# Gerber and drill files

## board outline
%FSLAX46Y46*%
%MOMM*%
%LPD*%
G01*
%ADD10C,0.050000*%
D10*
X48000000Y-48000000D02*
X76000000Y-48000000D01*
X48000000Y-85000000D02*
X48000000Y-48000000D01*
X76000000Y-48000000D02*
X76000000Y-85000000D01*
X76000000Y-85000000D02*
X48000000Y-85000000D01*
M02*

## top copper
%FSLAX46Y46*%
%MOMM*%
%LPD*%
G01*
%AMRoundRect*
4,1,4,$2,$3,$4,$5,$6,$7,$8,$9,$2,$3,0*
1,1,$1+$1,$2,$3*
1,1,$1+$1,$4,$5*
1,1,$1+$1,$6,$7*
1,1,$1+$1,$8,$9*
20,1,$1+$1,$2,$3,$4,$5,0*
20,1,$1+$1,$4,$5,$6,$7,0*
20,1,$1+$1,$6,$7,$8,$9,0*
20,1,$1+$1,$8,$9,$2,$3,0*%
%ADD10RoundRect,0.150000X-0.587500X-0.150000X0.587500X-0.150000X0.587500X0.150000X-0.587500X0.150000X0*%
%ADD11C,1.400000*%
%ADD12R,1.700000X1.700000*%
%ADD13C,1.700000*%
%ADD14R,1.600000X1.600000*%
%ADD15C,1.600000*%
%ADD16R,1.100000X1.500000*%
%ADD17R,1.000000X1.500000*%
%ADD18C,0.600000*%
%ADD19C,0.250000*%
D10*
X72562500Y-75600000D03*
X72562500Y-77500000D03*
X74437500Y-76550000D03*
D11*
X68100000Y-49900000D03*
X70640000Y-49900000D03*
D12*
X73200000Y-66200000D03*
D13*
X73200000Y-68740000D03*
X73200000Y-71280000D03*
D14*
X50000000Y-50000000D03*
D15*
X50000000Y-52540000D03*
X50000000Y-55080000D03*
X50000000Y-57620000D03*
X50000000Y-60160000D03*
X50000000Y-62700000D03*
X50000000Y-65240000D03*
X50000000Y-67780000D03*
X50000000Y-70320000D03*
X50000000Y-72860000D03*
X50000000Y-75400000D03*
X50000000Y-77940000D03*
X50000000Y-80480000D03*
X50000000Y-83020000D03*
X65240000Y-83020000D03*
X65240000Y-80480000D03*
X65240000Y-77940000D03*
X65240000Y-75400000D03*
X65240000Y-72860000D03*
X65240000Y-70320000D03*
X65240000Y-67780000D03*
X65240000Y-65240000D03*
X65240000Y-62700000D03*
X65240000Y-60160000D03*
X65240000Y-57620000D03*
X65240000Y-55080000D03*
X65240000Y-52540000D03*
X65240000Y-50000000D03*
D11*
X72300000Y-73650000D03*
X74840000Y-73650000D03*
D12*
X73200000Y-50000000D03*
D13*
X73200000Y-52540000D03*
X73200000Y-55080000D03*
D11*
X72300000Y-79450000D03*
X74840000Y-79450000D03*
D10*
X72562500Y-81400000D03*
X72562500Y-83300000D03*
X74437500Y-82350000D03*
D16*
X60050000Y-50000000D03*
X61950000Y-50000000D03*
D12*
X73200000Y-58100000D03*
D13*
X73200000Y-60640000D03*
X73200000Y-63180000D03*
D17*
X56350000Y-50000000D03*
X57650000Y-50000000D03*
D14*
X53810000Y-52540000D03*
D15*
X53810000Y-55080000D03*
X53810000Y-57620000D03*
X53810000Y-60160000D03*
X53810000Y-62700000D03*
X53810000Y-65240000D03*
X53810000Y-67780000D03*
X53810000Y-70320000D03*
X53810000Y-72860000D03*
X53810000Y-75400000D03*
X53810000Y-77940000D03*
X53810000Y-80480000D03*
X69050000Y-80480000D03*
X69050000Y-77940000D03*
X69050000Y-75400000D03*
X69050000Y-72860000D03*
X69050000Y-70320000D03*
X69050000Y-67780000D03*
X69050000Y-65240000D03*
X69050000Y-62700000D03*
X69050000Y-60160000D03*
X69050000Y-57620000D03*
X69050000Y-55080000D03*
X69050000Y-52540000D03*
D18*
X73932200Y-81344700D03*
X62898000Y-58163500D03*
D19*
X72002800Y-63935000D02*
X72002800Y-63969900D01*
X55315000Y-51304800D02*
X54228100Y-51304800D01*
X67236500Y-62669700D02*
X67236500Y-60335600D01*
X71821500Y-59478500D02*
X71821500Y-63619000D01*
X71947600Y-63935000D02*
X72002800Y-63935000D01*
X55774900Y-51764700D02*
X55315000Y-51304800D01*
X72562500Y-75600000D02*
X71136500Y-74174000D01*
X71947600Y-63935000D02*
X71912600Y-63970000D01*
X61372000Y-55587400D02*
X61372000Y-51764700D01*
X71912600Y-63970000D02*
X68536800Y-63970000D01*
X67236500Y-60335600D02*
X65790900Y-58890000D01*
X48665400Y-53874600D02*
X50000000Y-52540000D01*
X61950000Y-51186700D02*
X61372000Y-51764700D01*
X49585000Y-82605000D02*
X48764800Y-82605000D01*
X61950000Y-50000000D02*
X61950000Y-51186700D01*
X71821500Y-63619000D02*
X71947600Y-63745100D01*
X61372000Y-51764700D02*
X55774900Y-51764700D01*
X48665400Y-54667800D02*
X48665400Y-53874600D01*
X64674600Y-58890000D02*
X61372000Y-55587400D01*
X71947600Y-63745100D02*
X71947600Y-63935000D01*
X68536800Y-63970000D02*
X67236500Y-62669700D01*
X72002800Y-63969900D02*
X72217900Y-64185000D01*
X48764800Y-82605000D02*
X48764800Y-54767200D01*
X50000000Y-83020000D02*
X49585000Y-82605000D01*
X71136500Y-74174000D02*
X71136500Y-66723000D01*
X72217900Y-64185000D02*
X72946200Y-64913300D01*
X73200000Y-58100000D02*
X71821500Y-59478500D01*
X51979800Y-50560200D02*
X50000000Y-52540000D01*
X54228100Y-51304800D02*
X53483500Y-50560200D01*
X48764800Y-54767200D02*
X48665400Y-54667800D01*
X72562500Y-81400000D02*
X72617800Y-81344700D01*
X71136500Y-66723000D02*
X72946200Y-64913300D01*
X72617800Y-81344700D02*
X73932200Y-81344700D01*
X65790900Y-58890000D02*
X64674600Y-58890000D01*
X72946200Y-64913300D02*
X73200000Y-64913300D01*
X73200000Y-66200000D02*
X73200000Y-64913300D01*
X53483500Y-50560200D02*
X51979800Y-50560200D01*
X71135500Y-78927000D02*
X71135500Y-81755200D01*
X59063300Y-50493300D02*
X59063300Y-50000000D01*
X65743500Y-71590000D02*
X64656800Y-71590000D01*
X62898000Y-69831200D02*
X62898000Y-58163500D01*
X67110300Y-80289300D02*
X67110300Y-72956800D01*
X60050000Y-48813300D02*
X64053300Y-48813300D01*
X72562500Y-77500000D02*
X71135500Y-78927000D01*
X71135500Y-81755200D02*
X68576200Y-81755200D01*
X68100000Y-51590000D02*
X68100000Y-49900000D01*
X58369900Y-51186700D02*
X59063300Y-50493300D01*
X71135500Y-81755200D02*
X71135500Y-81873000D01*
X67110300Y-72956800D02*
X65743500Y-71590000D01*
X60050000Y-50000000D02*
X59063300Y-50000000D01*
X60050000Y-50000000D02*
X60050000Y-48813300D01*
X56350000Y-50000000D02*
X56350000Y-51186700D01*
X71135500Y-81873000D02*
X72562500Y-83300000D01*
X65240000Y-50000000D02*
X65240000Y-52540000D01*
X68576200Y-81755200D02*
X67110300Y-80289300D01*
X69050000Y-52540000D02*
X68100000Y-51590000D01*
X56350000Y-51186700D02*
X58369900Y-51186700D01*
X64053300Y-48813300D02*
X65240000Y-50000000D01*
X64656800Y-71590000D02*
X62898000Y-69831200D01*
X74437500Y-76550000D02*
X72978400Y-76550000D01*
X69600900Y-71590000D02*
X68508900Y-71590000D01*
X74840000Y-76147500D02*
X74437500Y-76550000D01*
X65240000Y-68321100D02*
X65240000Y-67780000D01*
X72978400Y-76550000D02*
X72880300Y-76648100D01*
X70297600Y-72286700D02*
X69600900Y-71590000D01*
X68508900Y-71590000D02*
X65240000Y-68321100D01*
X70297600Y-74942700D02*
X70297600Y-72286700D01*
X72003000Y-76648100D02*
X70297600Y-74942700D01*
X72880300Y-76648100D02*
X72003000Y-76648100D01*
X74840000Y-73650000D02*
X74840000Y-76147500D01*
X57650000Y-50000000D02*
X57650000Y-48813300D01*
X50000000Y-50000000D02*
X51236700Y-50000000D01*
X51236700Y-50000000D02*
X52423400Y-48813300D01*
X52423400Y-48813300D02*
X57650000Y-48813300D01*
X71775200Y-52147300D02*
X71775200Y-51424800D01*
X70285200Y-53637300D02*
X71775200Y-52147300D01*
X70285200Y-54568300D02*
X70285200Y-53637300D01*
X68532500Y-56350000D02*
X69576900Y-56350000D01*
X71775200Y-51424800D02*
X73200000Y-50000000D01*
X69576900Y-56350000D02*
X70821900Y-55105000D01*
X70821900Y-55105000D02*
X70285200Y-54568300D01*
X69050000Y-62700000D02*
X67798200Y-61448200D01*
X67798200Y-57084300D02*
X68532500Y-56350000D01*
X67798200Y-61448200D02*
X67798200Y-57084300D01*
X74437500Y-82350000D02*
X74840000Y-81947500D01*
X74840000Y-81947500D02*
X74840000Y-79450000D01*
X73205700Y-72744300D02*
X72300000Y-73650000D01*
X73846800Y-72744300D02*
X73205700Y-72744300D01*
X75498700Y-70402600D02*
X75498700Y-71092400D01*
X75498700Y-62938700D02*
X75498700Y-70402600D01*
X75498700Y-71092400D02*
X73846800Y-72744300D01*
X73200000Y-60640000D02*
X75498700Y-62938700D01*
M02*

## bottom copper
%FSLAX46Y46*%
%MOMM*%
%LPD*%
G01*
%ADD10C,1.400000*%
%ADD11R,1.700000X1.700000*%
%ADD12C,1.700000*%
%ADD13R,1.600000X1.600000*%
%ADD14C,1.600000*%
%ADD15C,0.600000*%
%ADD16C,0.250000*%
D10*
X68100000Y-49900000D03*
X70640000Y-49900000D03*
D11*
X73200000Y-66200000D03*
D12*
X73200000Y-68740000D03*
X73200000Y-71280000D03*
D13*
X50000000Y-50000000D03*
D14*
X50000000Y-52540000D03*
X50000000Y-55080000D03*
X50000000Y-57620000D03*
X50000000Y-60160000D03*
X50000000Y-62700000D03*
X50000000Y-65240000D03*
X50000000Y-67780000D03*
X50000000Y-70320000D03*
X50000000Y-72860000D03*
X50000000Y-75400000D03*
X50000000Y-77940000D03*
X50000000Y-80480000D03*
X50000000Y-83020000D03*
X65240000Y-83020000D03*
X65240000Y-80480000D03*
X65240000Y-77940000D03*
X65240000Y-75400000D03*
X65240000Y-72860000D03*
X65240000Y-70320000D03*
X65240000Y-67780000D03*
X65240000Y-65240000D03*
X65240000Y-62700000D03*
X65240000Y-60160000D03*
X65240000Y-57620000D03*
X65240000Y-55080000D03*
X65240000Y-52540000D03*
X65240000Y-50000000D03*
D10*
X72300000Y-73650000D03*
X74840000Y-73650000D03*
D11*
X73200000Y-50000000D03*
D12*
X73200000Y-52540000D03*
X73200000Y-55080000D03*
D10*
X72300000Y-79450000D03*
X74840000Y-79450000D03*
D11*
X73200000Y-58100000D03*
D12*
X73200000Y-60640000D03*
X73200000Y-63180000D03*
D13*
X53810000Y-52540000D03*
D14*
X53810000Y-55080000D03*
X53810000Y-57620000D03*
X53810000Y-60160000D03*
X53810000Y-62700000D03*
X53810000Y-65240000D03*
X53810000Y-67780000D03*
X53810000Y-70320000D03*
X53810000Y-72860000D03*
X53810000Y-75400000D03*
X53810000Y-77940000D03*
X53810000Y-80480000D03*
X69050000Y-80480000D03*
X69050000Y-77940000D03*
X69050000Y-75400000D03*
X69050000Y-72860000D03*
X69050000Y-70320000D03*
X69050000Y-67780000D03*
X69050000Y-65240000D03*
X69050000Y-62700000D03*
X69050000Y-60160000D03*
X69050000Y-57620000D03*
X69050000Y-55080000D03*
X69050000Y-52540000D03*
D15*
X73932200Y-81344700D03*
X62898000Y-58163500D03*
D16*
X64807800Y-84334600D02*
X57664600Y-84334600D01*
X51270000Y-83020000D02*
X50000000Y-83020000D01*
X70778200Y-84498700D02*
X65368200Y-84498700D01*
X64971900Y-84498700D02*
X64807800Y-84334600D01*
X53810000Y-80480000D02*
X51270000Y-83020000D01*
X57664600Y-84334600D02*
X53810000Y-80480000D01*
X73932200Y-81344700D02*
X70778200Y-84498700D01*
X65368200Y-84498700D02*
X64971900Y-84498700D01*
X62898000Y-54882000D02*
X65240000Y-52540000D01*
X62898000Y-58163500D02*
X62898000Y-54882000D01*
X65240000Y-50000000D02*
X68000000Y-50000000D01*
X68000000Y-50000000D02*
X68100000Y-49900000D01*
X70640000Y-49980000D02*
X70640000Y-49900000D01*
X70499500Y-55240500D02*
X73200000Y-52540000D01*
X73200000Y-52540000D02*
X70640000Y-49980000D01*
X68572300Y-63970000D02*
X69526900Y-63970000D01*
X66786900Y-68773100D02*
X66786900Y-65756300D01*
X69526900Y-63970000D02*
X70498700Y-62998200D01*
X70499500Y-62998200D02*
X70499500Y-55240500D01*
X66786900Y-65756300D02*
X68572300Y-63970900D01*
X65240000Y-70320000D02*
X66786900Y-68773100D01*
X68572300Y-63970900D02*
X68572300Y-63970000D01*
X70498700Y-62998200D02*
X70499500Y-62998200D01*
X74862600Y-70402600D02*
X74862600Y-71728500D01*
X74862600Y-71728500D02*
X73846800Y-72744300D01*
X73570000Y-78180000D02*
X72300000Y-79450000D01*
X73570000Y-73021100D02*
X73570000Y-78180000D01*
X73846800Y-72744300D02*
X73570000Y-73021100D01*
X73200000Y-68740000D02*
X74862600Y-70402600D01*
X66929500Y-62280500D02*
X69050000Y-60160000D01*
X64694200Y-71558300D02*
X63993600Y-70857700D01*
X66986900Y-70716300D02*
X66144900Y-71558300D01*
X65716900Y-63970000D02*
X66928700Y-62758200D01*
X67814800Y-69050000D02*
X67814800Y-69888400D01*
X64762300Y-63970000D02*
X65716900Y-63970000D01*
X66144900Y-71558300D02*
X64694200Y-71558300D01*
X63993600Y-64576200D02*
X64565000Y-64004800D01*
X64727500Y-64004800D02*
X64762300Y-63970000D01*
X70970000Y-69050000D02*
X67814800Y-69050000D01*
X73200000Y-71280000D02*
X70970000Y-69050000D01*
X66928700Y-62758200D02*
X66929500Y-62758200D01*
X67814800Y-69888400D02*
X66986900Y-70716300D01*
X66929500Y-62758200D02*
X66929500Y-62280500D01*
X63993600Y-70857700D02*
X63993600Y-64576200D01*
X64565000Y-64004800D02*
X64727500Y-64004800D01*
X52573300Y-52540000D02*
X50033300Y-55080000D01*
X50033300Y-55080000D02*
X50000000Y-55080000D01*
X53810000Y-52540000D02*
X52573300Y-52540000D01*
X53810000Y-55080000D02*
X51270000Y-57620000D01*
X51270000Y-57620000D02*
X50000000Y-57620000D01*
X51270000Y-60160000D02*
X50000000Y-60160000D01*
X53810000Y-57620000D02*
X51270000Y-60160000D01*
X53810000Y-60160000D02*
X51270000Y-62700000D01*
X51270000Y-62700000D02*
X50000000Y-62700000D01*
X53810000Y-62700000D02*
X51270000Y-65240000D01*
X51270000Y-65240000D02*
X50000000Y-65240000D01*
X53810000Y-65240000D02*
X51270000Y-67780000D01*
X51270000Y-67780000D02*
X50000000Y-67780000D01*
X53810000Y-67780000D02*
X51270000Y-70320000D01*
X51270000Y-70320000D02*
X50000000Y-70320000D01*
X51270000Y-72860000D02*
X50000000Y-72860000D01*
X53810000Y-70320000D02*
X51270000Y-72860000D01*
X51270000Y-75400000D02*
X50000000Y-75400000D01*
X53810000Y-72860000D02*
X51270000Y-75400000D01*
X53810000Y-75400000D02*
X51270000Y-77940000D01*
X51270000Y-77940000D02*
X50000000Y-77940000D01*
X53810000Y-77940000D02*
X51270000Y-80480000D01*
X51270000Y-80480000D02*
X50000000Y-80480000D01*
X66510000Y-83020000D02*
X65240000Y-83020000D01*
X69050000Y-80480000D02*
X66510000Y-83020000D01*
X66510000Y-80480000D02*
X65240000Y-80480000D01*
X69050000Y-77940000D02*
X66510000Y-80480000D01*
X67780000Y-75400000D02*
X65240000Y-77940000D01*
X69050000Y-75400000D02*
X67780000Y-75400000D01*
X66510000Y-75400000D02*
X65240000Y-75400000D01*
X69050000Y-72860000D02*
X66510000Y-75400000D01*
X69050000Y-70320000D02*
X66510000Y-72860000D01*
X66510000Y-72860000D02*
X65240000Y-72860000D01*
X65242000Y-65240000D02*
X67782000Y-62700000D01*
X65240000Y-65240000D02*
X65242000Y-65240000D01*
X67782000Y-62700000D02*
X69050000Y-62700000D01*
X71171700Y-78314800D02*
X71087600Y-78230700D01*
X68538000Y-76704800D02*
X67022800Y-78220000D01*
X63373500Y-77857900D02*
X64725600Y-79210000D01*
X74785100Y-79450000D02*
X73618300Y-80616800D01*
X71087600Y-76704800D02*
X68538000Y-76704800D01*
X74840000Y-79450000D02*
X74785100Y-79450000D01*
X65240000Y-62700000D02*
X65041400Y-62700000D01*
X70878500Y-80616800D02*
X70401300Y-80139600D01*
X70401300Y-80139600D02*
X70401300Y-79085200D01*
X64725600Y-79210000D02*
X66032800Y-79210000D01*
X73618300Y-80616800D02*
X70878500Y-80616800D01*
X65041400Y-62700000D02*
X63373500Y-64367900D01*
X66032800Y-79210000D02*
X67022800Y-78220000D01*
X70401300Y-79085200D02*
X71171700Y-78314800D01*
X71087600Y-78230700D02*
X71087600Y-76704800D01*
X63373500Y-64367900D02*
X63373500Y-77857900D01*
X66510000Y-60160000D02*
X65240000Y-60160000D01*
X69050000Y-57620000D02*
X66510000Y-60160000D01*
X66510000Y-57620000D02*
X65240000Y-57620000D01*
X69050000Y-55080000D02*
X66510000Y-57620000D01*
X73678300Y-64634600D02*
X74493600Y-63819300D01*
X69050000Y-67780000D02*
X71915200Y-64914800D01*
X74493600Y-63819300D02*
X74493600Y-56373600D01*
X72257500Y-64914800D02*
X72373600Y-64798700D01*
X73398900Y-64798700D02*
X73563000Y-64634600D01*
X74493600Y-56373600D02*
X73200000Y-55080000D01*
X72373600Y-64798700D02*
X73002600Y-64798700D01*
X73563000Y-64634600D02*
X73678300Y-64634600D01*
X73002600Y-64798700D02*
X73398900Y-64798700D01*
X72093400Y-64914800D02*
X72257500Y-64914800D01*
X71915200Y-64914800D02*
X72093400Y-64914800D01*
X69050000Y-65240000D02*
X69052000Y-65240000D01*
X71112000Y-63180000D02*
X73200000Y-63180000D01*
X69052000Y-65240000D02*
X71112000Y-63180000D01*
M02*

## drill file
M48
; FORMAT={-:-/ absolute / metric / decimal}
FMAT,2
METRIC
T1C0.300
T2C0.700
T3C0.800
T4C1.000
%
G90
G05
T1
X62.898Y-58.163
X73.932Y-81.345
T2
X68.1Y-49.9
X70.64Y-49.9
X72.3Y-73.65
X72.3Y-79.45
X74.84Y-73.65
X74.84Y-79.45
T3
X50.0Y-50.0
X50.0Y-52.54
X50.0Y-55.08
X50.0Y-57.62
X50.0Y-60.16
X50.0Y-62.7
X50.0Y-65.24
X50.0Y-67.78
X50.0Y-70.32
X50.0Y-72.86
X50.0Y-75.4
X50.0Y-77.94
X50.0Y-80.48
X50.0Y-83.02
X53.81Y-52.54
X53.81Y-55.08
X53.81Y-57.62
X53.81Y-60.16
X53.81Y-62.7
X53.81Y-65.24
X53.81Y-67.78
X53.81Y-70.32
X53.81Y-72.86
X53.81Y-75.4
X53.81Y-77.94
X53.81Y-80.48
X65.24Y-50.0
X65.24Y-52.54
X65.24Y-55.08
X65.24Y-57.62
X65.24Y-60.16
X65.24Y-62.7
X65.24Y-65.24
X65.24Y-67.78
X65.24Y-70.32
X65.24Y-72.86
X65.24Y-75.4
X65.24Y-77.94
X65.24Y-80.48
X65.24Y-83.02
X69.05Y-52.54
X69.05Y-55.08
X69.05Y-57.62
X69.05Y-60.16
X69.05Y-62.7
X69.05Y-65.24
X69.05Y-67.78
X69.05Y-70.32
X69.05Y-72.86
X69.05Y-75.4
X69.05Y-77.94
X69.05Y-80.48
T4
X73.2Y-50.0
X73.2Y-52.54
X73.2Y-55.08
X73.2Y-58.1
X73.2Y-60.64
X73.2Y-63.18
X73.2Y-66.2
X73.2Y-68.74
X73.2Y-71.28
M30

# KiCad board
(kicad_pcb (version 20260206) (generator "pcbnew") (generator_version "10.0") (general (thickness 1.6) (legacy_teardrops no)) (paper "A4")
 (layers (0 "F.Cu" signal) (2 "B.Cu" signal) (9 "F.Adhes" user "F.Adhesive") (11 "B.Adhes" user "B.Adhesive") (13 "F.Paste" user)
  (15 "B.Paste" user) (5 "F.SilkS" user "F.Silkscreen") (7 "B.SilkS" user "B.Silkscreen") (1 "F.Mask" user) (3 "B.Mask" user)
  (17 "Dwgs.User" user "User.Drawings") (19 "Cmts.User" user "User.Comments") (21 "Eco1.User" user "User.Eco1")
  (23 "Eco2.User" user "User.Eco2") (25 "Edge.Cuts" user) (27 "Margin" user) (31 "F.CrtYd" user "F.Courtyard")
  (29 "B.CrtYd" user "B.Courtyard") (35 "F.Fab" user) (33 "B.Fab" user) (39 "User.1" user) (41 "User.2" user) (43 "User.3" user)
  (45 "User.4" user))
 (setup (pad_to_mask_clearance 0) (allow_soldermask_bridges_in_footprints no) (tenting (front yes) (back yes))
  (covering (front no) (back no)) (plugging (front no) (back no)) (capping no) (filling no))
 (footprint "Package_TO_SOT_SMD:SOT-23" (layer "F.Cu") (at 73.5 76.55)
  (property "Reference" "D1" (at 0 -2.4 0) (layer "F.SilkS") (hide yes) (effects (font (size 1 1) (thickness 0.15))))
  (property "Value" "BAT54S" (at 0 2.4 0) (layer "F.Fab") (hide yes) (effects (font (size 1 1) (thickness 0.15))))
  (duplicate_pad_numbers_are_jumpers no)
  (pad "1" smd roundrect (at -0.9375 -0.95) (size 1.475 0.6) (layers "F.Cu" "F.Mask" "F.Paste") (roundrect_rratio 0.25) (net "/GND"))
  (pad "2" smd roundrect (at -0.9375 0.95) (size 1.475 0.6) (layers "F.Cu" "F.Mask" "F.Paste") (roundrect_rratio 0.25) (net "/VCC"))
  (pad "3" smd roundrect (at 0.9375 0) (size 1.475 0.6) (layers "F.Cu" "F.Mask" "F.Paste") (roundrect_rratio 0.25) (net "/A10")))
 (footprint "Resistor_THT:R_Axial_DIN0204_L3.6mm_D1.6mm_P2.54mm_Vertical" (layer "F.Cu") (at 68.1 49.9)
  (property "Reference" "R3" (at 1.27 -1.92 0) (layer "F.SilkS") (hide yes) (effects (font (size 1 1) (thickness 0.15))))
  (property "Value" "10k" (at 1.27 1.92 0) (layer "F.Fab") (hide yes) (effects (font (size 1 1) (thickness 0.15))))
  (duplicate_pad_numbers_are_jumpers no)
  (pad "1" thru_hole circle (at 0 0) (size 1.4 1.4) (drill 0.7) (layers "*.Cu" "*.Mask") (remove_unused_layers no) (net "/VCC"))
  (pad "2" thru_hole circle (at 2.54 0) (size 1.4 1.4) (drill 0.7) (layers "*.Cu" "*.Mask") (remove_unused_layers no) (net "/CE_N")))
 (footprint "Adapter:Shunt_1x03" (layer "F.Cu") (at 73.2 66.2)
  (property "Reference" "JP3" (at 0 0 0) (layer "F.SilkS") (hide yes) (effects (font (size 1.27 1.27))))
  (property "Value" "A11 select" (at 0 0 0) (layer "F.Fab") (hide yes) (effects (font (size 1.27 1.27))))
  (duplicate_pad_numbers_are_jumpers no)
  (pad "1" thru_hole rect (at 0 0) (size 1.7 1.7) (drill 1) (layers "*.Cu" "*.Mask") (remove_unused_layers no) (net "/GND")
   (thermal_bridge_angle 45))
  (pad "2" thru_hole circle (at 0 2.54) (size 1.7 1.7) (drill 1) (layers "*.Cu" "*.Mask") (remove_unused_layers no) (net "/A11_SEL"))
  (pad "3" thru_hole circle (at 0 5.08) (size 1.7 1.7) (drill 1) (layers "*.Cu" "*.Mask") (remove_unused_layers no) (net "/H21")))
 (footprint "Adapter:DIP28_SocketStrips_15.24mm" (layer "F.Cu") (at 50 50)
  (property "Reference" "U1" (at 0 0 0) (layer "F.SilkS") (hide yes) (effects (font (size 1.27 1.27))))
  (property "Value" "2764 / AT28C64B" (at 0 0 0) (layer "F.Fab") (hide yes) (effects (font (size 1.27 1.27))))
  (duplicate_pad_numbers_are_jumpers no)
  (pad "1" thru_hole rect (at 0 0) (size 1.6 1.6) (drill 0.8) (layers "*.Cu" "*.Mask") (remove_unused_layers no) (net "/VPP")
   (thermal_bridge_angle 45))
  (pad "2" thru_hole circle (at 0 2.54) (size 1.6 1.6) (drill 0.8) (layers "*.Cu" "*.Mask") (remove_unused_layers no) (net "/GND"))
  (pad "3" thru_hole circle (at 0 5.08) (size 1.6 1.6) (drill 0.8) (layers "*.Cu" "*.Mask") (remove_unused_layers no) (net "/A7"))
  (pad "4" thru_hole circle (at 0 7.62) (size 1.6 1.6) (drill 0.8) (layers "*.Cu" "*.Mask") (remove_unused_layers no) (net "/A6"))
  (pad "5" thru_hole circle (at 0 10.16) (size 1.6 1.6) (drill 0.8) (layers "*.Cu" "*.Mask") (remove_unused_layers no) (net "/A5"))
  (pad "6" thru_hole circle (at 0 12.7) (size 1.6 1.6) (drill 0.8) (layers "*.Cu" "*.Mask") (remove_unused_layers no) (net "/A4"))
  (pad "7" thru_hole circle (at 0 15.24) (size 1.6 1.6) (drill 0.8) (layers "*.Cu" "*.Mask") (remove_unused_layers no) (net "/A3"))
  (pad "8" thru_hole circle (at 0 17.78) (size 1.6 1.6) (drill 0.8) (layers "*.Cu" "*.Mask") (remove_unused_layers no) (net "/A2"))
  (pad "9" thru_hole circle (at 0 20.32) (size 1.6 1.6) (drill 0.8) (layers "*.Cu" "*.Mask") (remove_unused_layers no) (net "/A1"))
  (pad "10" thru_hole circle (at 0 22.86) (size 1.6 1.6) (drill 0.8) (layers "*.Cu" "*.Mask") (remove_unused_layers no) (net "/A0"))
  (pad "11" thru_hole circle (at 0 25.4) (size 1.6 1.6) (drill 0.8) (layers "*.Cu" "*.Mask") (remove_unused_layers no) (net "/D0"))
  (pad "12" thru_hole circle (at 0 27.94) (size 1.6 1.6) (drill 0.8) (layers "*.Cu" "*.Mask") (remove_unused_layers no) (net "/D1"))
  (pad "13" thru_hole circle (at 0 30.48) (size 1.6 1.6) (drill 0.8) (layers "*.Cu" "*.Mask") (remove_unused_layers no) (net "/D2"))
  (pad "14" thru_hole circle (at 0 33.02) (size 1.6 1.6) (drill 0.8) (layers "*.Cu" "*.Mask") (remove_unused_layers no) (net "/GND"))
  (pad "15" thru_hole circle (at 15.24 33.02) (size 1.6 1.6) (drill 0.8) (layers "*.Cu" "*.Mask") (remove_unused_layers no) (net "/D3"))
  (pad "16" thru_hole circle (at 15.24 30.48) (size 1.6 1.6) (drill 0.8) (layers "*.Cu" "*.Mask") (remove_unused_layers no) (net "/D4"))
  (pad "17" thru_hole circle (at 15.24 27.94) (size 1.6 1.6) (drill 0.8) (layers "*.Cu" "*.Mask") (remove_unused_layers no) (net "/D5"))
  (pad "18" thru_hole circle (at 15.24 25.4) (size 1.6 1.6) (drill 0.8) (layers "*.Cu" "*.Mask") (remove_unused_layers no) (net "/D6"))
  (pad "19" thru_hole circle (at 15.24 22.86) (size 1.6 1.6) (drill 0.8) (layers "*.Cu" "*.Mask") (remove_unused_layers no) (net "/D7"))
  (pad "20" thru_hole circle (at 15.24 20.32) (size 1.6 1.6) (drill 0.8) (layers "*.Cu" "*.Mask") (remove_unused_layers no) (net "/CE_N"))
  (pad "21" thru_hole circle (at 15.24 17.78) (size 1.6 1.6) (drill 0.8) (layers "*.Cu" "*.Mask") (remove_unused_layers no) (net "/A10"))
  (pad "22" thru_hole circle (at 15.24 15.24) (size 1.6 1.6) (drill 0.8) (layers "*.Cu" "*.Mask") (remove_unused_layers no) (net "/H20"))
  (pad "23" thru_hole circle (at 15.24 12.7) (size 1.6 1.6) (drill 0.8) (layers "*.Cu" "*.Mask") (remove_unused_layers no) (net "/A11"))
  (pad "24" thru_hole circle (at 15.24 10.16) (size 1.6 1.6) (drill 0.8) (layers "*.Cu" "*.Mask") (remove_unused_layers no) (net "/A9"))
  (pad "25" thru_hole circle (at 15.24 7.62) (size 1.6 1.6) (drill 0.8) (layers "*.Cu" "*.Mask") (remove_unused_layers no) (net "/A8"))
  (pad "26" thru_hole circle (at 15.24 5.08) (size 1.6 1.6) (drill 0.8) (layers "*.Cu" "*.Mask") (remove_unused_layers no)
   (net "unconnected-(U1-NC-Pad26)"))
  (pad "27" thru_hole circle (at 15.24 2.54) (size 1.6 1.6) (drill 0.8) (layers "*.Cu" "*.Mask") (remove_unused_layers no) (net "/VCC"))
  (pad "28" thru_hole circle (at 15.24 0) (size 1.6 1.6) (drill 0.8) (layers "*.Cu" "*.Mask") (remove_unused_layers no) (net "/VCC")))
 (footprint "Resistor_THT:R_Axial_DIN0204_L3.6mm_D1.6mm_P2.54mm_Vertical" (layer "F.Cu") (at 72.3 73.65)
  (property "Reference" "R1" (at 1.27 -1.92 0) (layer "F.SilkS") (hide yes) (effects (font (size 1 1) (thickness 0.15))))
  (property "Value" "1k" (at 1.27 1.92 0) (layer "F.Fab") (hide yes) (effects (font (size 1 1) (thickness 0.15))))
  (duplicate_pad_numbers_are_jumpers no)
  (pad "1" thru_hole circle (at 0 0) (size 1.4 1.4) (drill 0.7) (layers "*.Cu" "*.Mask") (remove_unused_layers no) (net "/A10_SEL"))
  (pad "2" thru_hole circle (at 2.54 0) (size 1.4 1.4) (drill 0.7) (layers "*.Cu" "*.Mask") (remove_unused_layers no) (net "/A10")))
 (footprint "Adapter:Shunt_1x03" (layer "F.Cu") (at 73.2 50)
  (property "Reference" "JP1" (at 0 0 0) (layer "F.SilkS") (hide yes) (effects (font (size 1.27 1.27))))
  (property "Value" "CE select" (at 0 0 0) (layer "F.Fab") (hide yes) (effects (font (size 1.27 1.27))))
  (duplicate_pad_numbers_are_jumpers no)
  (pad "1" thru_hole rect (at 0 0) (size 1.7 1.7) (drill 1) (layers "*.Cu" "*.Mask") (remove_unused_layers no) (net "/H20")
   (thermal_bridge_angle 45))
  (pad "2" thru_hole circle (at 0 2.54) (size 1.7 1.7) (drill 1) (layers "*.Cu" "*.Mask") (remove_unused_layers no) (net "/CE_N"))
  (pad "3" thru_hole circle (at 0 5.08) (size 1.7 1.7) (drill 1) (layers "*.Cu" "*.Mask") (remove_unused_layers no) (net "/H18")))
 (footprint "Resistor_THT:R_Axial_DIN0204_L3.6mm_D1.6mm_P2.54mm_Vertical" (layer "F.Cu") (at 72.3 79.45)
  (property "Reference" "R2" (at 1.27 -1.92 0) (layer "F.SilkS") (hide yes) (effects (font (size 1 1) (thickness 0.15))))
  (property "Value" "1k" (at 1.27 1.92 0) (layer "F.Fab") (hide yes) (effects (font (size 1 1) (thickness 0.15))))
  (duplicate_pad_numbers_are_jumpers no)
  (pad "1" thru_hole circle (at 0 0) (size 1.4 1.4) (drill 0.7) (layers "*.Cu" "*.Mask") (remove_unused_layers no) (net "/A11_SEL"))
  (pad "2" thru_hole circle (at 2.54 0) (size 1.4 1.4) (drill 0.7) (layers "*.Cu" "*.Mask") (remove_unused_layers no) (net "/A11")))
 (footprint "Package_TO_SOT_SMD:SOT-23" (layer "F.Cu") (at 73.5 82.35)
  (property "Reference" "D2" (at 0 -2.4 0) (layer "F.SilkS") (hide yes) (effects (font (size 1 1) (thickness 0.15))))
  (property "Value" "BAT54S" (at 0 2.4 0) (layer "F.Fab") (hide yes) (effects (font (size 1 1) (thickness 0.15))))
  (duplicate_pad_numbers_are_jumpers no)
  (pad "1" smd roundrect (at -0.9375 -0.95) (size 1.475 0.6) (layers "F.Cu" "F.Mask" "F.Paste") (roundrect_rratio 0.25) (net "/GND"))
  (pad "2" smd roundrect (at -0.9375 0.95) (size 1.475 0.6) (layers "F.Cu" "F.Mask" "F.Paste") (roundrect_rratio 0.25) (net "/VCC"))
  (pad "3" smd roundrect (at 0.9375 0) (size 1.475 0.6) (layers "F.Cu" "F.Mask" "F.Paste") (roundrect_rratio 0.25) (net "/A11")))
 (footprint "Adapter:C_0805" (layer "F.Cu") (at 61 50)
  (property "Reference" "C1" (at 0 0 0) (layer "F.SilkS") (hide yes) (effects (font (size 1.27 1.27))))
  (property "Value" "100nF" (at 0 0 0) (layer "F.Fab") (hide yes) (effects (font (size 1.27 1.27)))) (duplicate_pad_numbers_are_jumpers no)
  (pad "1" smd rect (at -0.95 0) (size 1.1 1.5) (layers "F.Cu" "F.Mask" "F.Paste") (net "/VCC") (thermal_bridge_angle 45))
  (pad "2" smd rect (at 0.95 0) (size 1.1 1.5) (layers "F.Cu" "F.Mask" "F.Paste") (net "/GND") (thermal_bridge_angle 45)))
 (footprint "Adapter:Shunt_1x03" (layer "F.Cu") (at 73.2 58.1)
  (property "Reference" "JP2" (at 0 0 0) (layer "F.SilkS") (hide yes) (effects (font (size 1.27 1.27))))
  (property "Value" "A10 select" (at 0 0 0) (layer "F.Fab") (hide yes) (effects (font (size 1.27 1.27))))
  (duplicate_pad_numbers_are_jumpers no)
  (pad "1" thru_hole rect (at 0 0) (size 1.7 1.7) (drill 1) (layers "*.Cu" "*.Mask") (remove_unused_layers no) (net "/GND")
   (thermal_bridge_angle 45))
  (pad "2" thru_hole circle (at 0 2.54) (size 1.7 1.7) (drill 1) (layers "*.Cu" "*.Mask") (remove_unused_layers no) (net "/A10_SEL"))
  (pad "3" thru_hole circle (at 0 5.08) (size 1.7 1.7) (drill 1) (layers "*.Cu" "*.Mask") (remove_unused_layers no) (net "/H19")))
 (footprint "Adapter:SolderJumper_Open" (layer "F.Cu") (at 57 50)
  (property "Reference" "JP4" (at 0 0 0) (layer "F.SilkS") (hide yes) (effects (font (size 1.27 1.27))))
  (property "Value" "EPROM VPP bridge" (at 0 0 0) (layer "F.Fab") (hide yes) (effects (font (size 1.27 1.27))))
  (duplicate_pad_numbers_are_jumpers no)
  (pad "1" smd rect (at -0.65 0) (size 1 1.5) (layers "F.Cu" "F.Mask") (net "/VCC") (thermal_bridge_angle 45))
  (pad "2" smd rect (at 0.65 0) (size 1 1.5) (layers "F.Cu" "F.Mask") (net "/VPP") (thermal_bridge_angle 45)))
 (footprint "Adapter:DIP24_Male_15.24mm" (layer "B.Cu") (at 53.81 52.54)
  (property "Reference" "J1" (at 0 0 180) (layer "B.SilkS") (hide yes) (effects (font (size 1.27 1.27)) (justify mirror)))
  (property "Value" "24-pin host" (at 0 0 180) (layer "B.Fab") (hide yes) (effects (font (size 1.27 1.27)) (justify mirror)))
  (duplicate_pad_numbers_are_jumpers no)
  (pad "1" thru_hole rect (at 0 0) (size 1.6 1.6) (drill 0.8) (layers "*.Cu" "*.Mask") (remove_unused_layers no) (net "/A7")
   (thermal_bridge_angle 45))
  (pad "2" thru_hole circle (at 0 2.54) (size 1.6 1.6) (drill 0.8) (layers "*.Cu" "*.Mask") (remove_unused_layers no) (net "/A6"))
  (pad "3" thru_hole circle (at 0 5.08) (size 1.6 1.6) (drill 0.8) (layers "*.Cu" "*.Mask") (remove_unused_layers no) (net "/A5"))
  (pad "4" thru_hole circle (at 0 7.62) (size 1.6 1.6) (drill 0.8) (layers "*.Cu" "*.Mask") (remove_unused_layers no) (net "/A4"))
  (pad "5" thru_hole circle (at 0 10.16) (size 1.6 1.6) (drill 0.8) (layers "*.Cu" "*.Mask") (remove_unused_layers no) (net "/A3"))
  (pad "6" thru_hole circle (at 0 12.7) (size 1.6 1.6) (drill 0.8) (layers "*.Cu" "*.Mask") (remove_unused_layers no) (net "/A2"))
  (pad "7" thru_hole circle (at 0 15.24) (size 1.6 1.6) (drill 0.8) (layers "*.Cu" "*.Mask") (remove_unused_layers no) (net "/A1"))
  (pad "8" thru_hole circle (at 0 17.78) (size 1.6 1.6) (drill 0.8) (layers "*.Cu" "*.Mask") (remove_unused_layers no) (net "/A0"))
  (pad "9" thru_hole circle (at 0 20.32) (size 1.6 1.6) (drill 0.8) (layers "*.Cu" "*.Mask") (remove_unused_layers no) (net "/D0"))
  (pad "10" thru_hole circle (at 0 22.86) (size 1.6 1.6) (drill 0.8) (layers "*.Cu" "*.Mask") (remove_unused_layers no) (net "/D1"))
  (pad "11" thru_hole circle (at 0 25.4) (size 1.6 1.6) (drill 0.8) (layers "*.Cu" "*.Mask") (remove_unused_layers no) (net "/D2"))
  (pad "12" thru_hole circle (at 0 27.94) (size 1.6 1.6) (drill 0.8) (layers "*.Cu" "*.Mask") (remove_unused_layers no) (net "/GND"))
  (pad "13" thru_hole circle (at 15.24 27.94) (size 1.6 1.6) (drill 0.8) (layers "*.Cu" "*.Mask") (remove_unused_layers no) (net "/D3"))
  (pad "14" thru_hole circle (at 15.24 25.4) (size 1.6 1.6) (drill 0.8) (layers "*.Cu" "*.Mask") (remove_unused_layers no) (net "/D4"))
  (pad "15" thru_hole circle (at 15.24 22.86) (size 1.6 1.6) (drill 0.8) (layers "*.Cu" "*.Mask") (remove_unused_layers no) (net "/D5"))
  (pad "16" thru_hole circle (at 15.24 20.32) (size 1.6 1.6) (drill 0.8) (layers "*.Cu" "*.Mask") (remove_unused_layers no) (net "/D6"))
  (pad "17" thru_hole circle (at 15.24 17.78) (size 1.6 1.6) (drill 0.8) (layers "*.Cu" "*.Mask") (remove_unused_layers no) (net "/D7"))
  (pad "18" thru_hole circle (at 15.24 15.24) (size 1.6 1.6) (drill 0.8) (layers "*.Cu" "*.Mask") (remove_unused_layers no) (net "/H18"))
  (pad "19" thru_hole circle (at 15.24 12.7) (size 1.6 1.6) (drill 0.8) (layers "*.Cu" "*.Mask") (remove_unused_layers no) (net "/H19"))
  (pad "20" thru_hole circle (at 15.24 10.16) (size 1.6 1.6) (drill 0.8) (layers "*.Cu" "*.Mask") (remove_unused_layers no) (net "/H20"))
  (pad "21" thru_hole circle (at 15.24 7.62) (size 1.6 1.6) (drill 0.8) (layers "*.Cu" "*.Mask") (remove_unused_layers no) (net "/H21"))
  (pad "22" thru_hole circle (at 15.24 5.08) (size 1.6 1.6) (drill 0.8) (layers "*.Cu" "*.Mask") (remove_unused_layers no) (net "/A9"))
  (pad "23" thru_hole circle (at 15.24 2.54) (size 1.6 1.6) (drill 0.8) (layers "*.Cu" "*.Mask") (remove_unused_layers no) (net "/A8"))
  (pad "24" thru_hole circle (at 15.24 0) (size 1.6 1.6) (drill 0.8) (layers "*.Cu" "*.Mask") (remove_unused_layers no) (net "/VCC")))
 (gr_line (start 48 48) (end 76 48) (stroke (width 0.05) (type default)) (layer "Edge.Cuts"))
 (gr_line (start 48 85) (end 48 48) (stroke (width 0.05) (type default)) (layer "Edge.Cuts"))
 (gr_line (start 76 48) (end 76 85) (stroke (width 0.05) (type default)) (layer "Edge.Cuts"))
 (gr_line (start 76 85) (end 48 85) (stroke (width 0.05) (type default)) (layer "Edge.Cuts"))
 (segment (start 72.0028 63.935) (end 72.0028 63.9699) (width 0.25) (layer "F.Cu") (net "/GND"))
 (segment (start 55.315 51.3048) (end 54.2281 51.3048) (width 0.25) (layer "F.Cu") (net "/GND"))
 (segment (start 67.2365 62.6697) (end 67.2365 60.3356) (width 0.25) (layer "F.Cu") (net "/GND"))
 (segment (start 71.8215 59.4785) (end 71.8215 63.619) (width 0.25) (layer "F.Cu") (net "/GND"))
 (segment (start 71.9476 63.935) (end 72.0028 63.935) (width 0.25) (layer "F.Cu") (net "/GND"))
 (segment (start 55.7749 51.7647) (end 55.315 51.3048) (width 0.25) (layer "F.Cu") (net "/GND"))
 (segment (start 72.5625 75.6) (end 71.1365 74.174) (width 0.25) (layer "F.Cu") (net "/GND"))
 (segment (start 71.9476 63.935) (end 71.9126 63.97) (width 0.25) (layer "F.Cu") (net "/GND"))
 (segment (start 61.372 55.5874) (end 61.372 51.7647) (width 0.25) (layer "F.Cu") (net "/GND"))
 (segment (start 71.9126 63.97) (end 68.5368 63.97) (width 0.25) (layer "F.Cu") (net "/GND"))
 (segment (start 67.2365 60.3356) (end 65.7909 58.89) (width 0.25) (layer "F.Cu") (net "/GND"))
 (segment (start 48.6654 53.8746) (end 50 52.54) (width 0.25) (layer "F.Cu") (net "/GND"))
 (segment (start 61.95 51.1867) (end 61.372 51.7647) (width 0.25) (layer "F.Cu") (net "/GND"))
 (segment (start 49.585 82.605) (end 48.7648 82.605) (width 0.25) (layer "F.Cu") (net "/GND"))
 (segment (start 61.95 50) (end 61.95 51.1867) (width 0.25) (layer "F.Cu") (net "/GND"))
 (segment (start 71.8215 63.619) (end 71.9476 63.7451) (width 0.25) (layer "F.Cu") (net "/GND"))
 (segment (start 61.372 51.7647) (end 55.7749 51.7647) (width 0.25) (layer "F.Cu") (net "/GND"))
 (segment (start 48.6654 54.6678) (end 48.6654 53.8746) (width 0.25) (layer "F.Cu") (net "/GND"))
 (segment (start 64.6746 58.89) (end 61.372 55.5874) (width 0.25) (layer "F.Cu") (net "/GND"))
 (segment (start 71.9476 63.7451) (end 71.9476 63.935) (width 0.25) (layer "F.Cu") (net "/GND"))
 (segment (start 68.5368 63.97) (end 67.2365 62.6697) (width 0.25) (layer "F.Cu") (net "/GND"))
 (segment (start 72.0028 63.9699) (end 72.2179 64.185) (width 0.25) (layer "F.Cu") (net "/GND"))
 (segment (start 48.7648 82.605) (end 48.7648 54.7672) (width 0.25) (layer "F.Cu") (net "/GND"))
 (segment (start 50 83.02) (end 49.585 82.605) (width 0.25) (layer "F.Cu") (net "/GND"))
 (segment (start 71.1365 74.174) (end 71.1365 66.723) (width 0.25) (layer "F.Cu") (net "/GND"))
 (segment (start 72.2179 64.185) (end 72.9462 64.9133) (width 0.25) (layer "F.Cu") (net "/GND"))
 (segment (start 73.2 58.1) (end 71.8215 59.4785) (width 0.25) (layer "F.Cu") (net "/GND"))
 (segment (start 51.9798 50.5602) (end 50 52.54) (width 0.25) (layer "F.Cu") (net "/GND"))
 (segment (start 54.2281 51.3048) (end 53.4835 50.5602) (width 0.25) (layer "F.Cu") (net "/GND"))
 (segment (start 48.7648 54.7672) (end 48.6654 54.6678) (width 0.25) (layer "F.Cu") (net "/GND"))
 (segment (start 72.5625 81.4) (end 72.6178 81.3447) (width 0.25) (layer "F.Cu") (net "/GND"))
 (segment (start 71.1365 66.723) (end 72.9462 64.9133) (width 0.25) (layer "F.Cu") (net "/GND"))
 (segment (start 72.6178 81.3447) (end 73.9322 81.3447) (width 0.25) (layer "F.Cu") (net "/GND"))
 (segment (start 65.7909 58.89) (end 64.6746 58.89) (width 0.25) (layer "F.Cu") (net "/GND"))
 (segment (start 72.9462 64.9133) (end 73.2 64.9133) (width 0.25) (layer "F.Cu") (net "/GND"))
 (segment (start 73.2 66.2) (end 73.2 64.9133) (width 0.25) (layer "F.Cu") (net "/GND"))
 (segment (start 53.4835 50.5602) (end 51.9798 50.5602) (width 0.25) (layer "F.Cu") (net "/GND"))
 (via (at 73.9322 81.3447) (size 0.6) (drill 0.3) (layers "F.Cu" "B.Cu") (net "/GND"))
 (segment (start 64.8078 84.3346) (end 57.6646 84.3346) (width 0.25) (layer "B.Cu") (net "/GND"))
 (segment (start 51.27 83.02) (end 50 83.02) (width 0.25) (layer "B.Cu") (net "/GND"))
 (segment (start 70.7782 84.4987) (end 65.3682 84.4987) (width 0.25) (layer "B.Cu") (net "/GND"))
 (segment (start 64.9719 84.4987) (end 64.8078 84.3346) (width 0.25) (layer "B.Cu") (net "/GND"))
 (segment (start 53.81 80.48) (end 51.27 83.02) (width 0.25) (layer "B.Cu") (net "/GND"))
 (segment (start 57.6646 84.3346) (end 53.81 80.48) (width 0.25) (layer "B.Cu") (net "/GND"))
 (segment (start 73.9322 81.3447) (end 70.7782 84.4987) (width 0.25) (layer "B.Cu") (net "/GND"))
 (segment (start 65.3682 84.4987) (end 64.9719 84.4987) (width 0.25) (layer "B.Cu") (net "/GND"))
 (segment (start 71.1355 78.927) (end 71.1355 81.7552) (width 0.25) (layer "F.Cu") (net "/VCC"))
 (segment (start 59.0633 50.4933) (end 59.0633 50) (width 0.25) (layer "F.Cu") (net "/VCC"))
 (segment (start 65.7435 71.59) (end 64.6568 71.59) (width 0.25) (layer "F.Cu") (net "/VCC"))
 (segment (start 62.898 69.8312) (end 62.898 58.1635) (width 0.25) (layer "F.Cu") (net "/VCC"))
 (segment (start 67.1103 80.2893) (end 67.1103 72.9568) (width 0.25) (layer "F.Cu") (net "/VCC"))
 (segment (start 60.05 48.8133) (end 64.0533 48.8133) (width 0.25) (layer "F.Cu") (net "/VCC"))
 (segment (start 72.5625 77.5) (end 71.1355 78.927) (width 0.25) (layer "F.Cu") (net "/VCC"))
 (segment (start 71.1355 81.7552) (end 68.5762 81.7552) (width 0.25) (layer "F.Cu") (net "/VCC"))
 (segment (start 68.1 51.59) (end 68.1 49.9) (width 0.25) (layer "F.Cu") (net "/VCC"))
 (segment (start 58.3699 51.1867) (end 59.0633 50.4933) (width 0.25) (layer "F.Cu") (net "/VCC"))
 (segment (start 71.1355 81.7552) (end 71.1355 81.873) (width 0.25) (layer "F.Cu") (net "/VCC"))
 (segment (start 67.1103 72.9568) (end 65.7435 71.59) (width 0.25) (layer "F.Cu") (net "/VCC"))
 (segment (start 60.05 50) (end 59.0633 50) (width 0.25) (layer "F.Cu") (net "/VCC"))
 (segment (start 60.05 50) (end 60.05 48.8133) (width 0.25) (layer "F.Cu") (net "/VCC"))
 (segment (start 56.35 50) (end 56.35 51.1867) (width 0.25) (layer "F.Cu") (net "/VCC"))
 (segment (start 71.1355 81.873) (end 72.5625 83.3) (width 0.25) (layer "F.Cu") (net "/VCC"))
 (segment (start 65.24 50) (end 65.24 52.54) (width 0.25) (layer "F.Cu") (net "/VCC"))
 (segment (start 68.5762 81.7552) (end 67.1103 80.2893) (width 0.25) (layer "F.Cu") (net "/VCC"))
 (segment (start 69.05 52.54) (end 68.1 51.59) (width 0.25) (layer "F.Cu") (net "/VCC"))
 (segment (start 56.35 51.1867) (end 58.3699 51.1867) (width 0.25) (layer "F.Cu") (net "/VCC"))
 (segment (start 64.0533 48.8133) (end 65.24 50) (width 0.25) (layer "F.Cu") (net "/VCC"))
 (segment (start 64.6568 71.59) (end 62.898 69.8312) (width 0.25) (layer "F.Cu") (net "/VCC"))
 (via (at 62.898 58.1635) (size 0.6) (drill 0.3) (layers "F.Cu" "B.Cu") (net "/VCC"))
 (segment (start 62.898 54.882) (end 65.24 52.54) (width 0.25) (layer "B.Cu") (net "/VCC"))
 (segment (start 62.898 58.1635) (end 62.898 54.882) (width 0.25) (layer "B.Cu") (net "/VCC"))
 (segment (start 65.24 50) (end 68 50) (width 0.25) (layer "B.Cu") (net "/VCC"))
 (segment (start 68 50) (end 68.1 49.9) (width 0.25) (layer "B.Cu") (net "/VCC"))
 (segment (start 74.4375 76.55) (end 72.9784 76.55) (width 0.25) (layer "F.Cu") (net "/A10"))
 (segment (start 69.6009 71.59) (end 68.5089 71.59) (width 0.25) (layer "F.Cu") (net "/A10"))
 (segment (start 74.84 76.1475) (end 74.4375 76.55) (width 0.25) (layer "F.Cu") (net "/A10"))
 (segment (start 65.24 68.3211) (end 65.24 67.78) (width 0.25) (layer "F.Cu") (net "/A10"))
 (segment (start 72.9784 76.55) (end 72.8803 76.6481) (width 0.25) (layer "F.Cu") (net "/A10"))
 (segment (start 70.2976 72.2867) (end 69.6009 71.59) (width 0.25) (layer "F.Cu") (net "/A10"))
 (segment (start 68.5089 71.59) (end 65.24 68.3211) (width 0.25) (layer "F.Cu") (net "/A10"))
 (segment (start 70.2976 74.9427) (end 70.2976 72.2867) (width 0.25) (layer "F.Cu") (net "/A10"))
 (segment (start 72.003 76.6481) (end 70.2976 74.9427) (width 0.25) (layer "F.Cu") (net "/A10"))
 (segment (start 72.8803 76.6481) (end 72.003 76.6481) (width 0.25) (layer "F.Cu") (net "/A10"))
 (segment (start 74.84 73.65) (end 74.84 76.1475) (width 0.25) (layer "F.Cu") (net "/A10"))
 (segment (start 70.64 49.98) (end 70.64 49.9) (width 0.25) (layer "B.Cu") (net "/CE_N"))
 (segment (start 70.4995 55.2405) (end 73.2 52.54) (width 0.25) (layer "B.Cu") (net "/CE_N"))
 (segment (start 73.2 52.54) (end 70.64 49.98) (width 0.25) (layer "B.Cu") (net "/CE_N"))
 (segment (start 68.5723 63.97) (end 69.5269 63.97) (width 0.25) (layer "B.Cu") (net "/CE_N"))
 (segment (start 66.7869 68.7731) (end 66.7869 65.7563) (width 0.25) (layer "B.Cu") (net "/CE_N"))
 (segment (start 69.5269 63.97) (end 70.4987 62.9982) (width 0.25) (layer "B.Cu") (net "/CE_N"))
 (segment (start 70.4995 62.9982) (end 70.4995 55.2405) (width 0.25) (layer "B.Cu") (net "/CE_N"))
 (segment (start 66.7869 65.7563) (end 68.5723 63.9709) (width 0.25) (layer "B.Cu") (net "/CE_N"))
 (segment (start 65.24 70.32) (end 66.7869 68.7731) (width 0.25) (layer "B.Cu") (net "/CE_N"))
 (segment (start 68.5723 63.9709) (end 68.5723 63.97) (width 0.25) (layer "B.Cu") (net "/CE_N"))
 (segment (start 70.4987 62.9982) (end 70.4995 62.9982) (width 0.25) (layer "B.Cu") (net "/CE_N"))
 (segment (start 74.8626 70.4026) (end 74.8626 71.7285) (width 0.25) (layer "B.Cu") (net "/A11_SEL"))
 (segment (start 74.8626 71.7285) (end 73.8468 72.7443) (width 0.25) (layer "B.Cu") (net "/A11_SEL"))
 (segment (start 73.57 78.18) (end 72.3 79.45) (width 0.25) (layer "B.Cu") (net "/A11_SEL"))
 (segment (start 73.57 73.0211) (end 73.57 78.18) (width 0.25) (layer "B.Cu") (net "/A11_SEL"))
 (segment (start 73.8468 72.7443) (end 73.57 73.0211) (width 0.25) (layer "B.Cu") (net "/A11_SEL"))
 (segment (start 73.2 68.74) (end 74.8626 70.4026) (width 0.25) (layer "B.Cu") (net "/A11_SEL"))
 (segment (start 66.9295 62.2805) (end 69.05 60.16) (width 0.25) (layer "B.Cu") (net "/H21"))
 (segment (start 64.6942 71.5583) (end 63.9936 70.8577) (width 0.25) (layer "B.Cu") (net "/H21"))
 (segment (start 66.9869 70.7163) (end 66.1449 71.5583) (width 0.25) (layer "B.Cu") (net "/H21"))
 (segment (start 65.7169 63.97) (end 66.9287 62.7582) (width 0.25) (layer "B.Cu") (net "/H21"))
 (segment (start 67.8148 69.05) (end 67.8148 69.8884) (width 0.25) (layer "B.Cu") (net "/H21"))
 (segment (start 64.7623 63.97) (end 65.7169 63.97) (width 0.25) (layer "B.Cu") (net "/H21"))
 (segment (start 66.1449 71.5583) (end 64.6942 71.5583) (width 0.25) (layer "B.Cu") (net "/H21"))
 (segment (start 63.9936 64.5762) (end 64.565 64.0048) (width 0.25) (layer "B.Cu") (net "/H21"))
 (segment (start 64.7275 64.0048) (end 64.7623 63.97) (width 0.25) (layer "B.Cu") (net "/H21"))
 (segment (start 70.97 69.05) (end 67.8148 69.05) (width 0.25) (layer "B.Cu") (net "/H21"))
 (segment (start 73.2 71.28) (end 70.97 69.05) (width 0.25) (layer "B.Cu") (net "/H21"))
 (segment (start 66.9287 62.7582) (end 66.9295 62.7582) (width 0.25) (layer "B.Cu") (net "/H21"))
 (segment (start 67.8148 69.8884) (end 66.9869 70.7163) (width 0.25) (layer "B.Cu") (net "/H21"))
 (segment (start 66.9295 62.7582) (end 66.9295 62.2805) (width 0.25) (layer "B.Cu") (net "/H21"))
 (segment (start 63.9936 70.8577) (end 63.9936 64.5762) (width 0.25) (layer "B.Cu") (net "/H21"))
 (segment (start 64.565 64.0048) (end 64.7275 64.0048) (width 0.25) (layer "B.Cu") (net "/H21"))
 (segment (start 57.65 50) (end 57.65 48.8133) (width 0.25) (layer "F.Cu") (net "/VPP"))
 (segment (start 50 50) (end 51.2367 50) (width 0.25) (layer "F.Cu") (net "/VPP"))
 (segment (start 51.2367 50) (end 52.4234 48.8133) (width 0.25) (layer "F.Cu") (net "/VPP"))
 (segment (start 52.4234 48.8133) (end 57.65 48.8133) (width 0.25) (layer "F.Cu") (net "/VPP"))
 (segment (start 52.5733 52.54) (end 50.0333 55.08) (width 0.25) (layer "B.Cu") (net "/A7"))
 (segment (start 50.0333 55.08) (end 50 55.08) (width 0.25) (layer "B.Cu") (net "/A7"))
 (segment (start 53.81 52.54) (end 52.5733 52.54) (width 0.25) (layer "B.Cu") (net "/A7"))
 (segment (start 53.81 55.08) (end 51.27 57.62) (width 0.25) (layer "B.Cu") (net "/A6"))
 (segment (start 51.27 57.62) (end 50 57.62) (width 0.25) (layer "B.Cu") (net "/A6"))
 (segment (start 51.27 60.16) (end 50 60.16) (width 0.25) (layer "B.Cu") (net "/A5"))
 (segment (start 53.81 57.62) (end 51.27 60.16) (width 0.25) (layer "B.Cu") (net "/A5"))
 (segment (start 53.81 60.16) (end 51.27 62.7) (width 0.25) (layer "B.Cu") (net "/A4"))
 (segment (start 51.27 62.7) (end 50 62.7) (width 0.25) (layer "B.Cu") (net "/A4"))
 (segment (start 53.81 62.7) (end 51.27 65.24) (width 0.25) (layer "B.Cu") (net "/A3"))
 (segment (start 51.27 65.24) (end 50 65.24) (width 0.25) (layer "B.Cu") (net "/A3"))
 (segment (start 53.81 65.24) (end 51.27 67.78) (width 0.25) (layer "B.Cu") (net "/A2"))
 (segment (start 51.27 67.78) (end 50 67.78) (width 0.25) (layer "B.Cu") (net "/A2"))
 (segment (start 53.81 67.78) (end 51.27 70.32) (width 0.25) (layer "B.Cu") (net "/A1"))
 (segment (start 51.27 70.32) (end 50 70.32) (width 0.25) (layer "B.Cu") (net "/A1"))
 (segment (start 51.27 72.86) (end 50 72.86) (width 0.25) (layer "B.Cu") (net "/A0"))
 (segment (start 53.81 70.32) (end 51.27 72.86) (width 0.25) (layer "B.Cu") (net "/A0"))
 (segment (start 51.27 75.4) (end 50 75.4) (width 0.25) (layer "B.Cu") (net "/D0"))
 (segment (start 53.81 72.86) (end 51.27 75.4) (width 0.25) (layer "B.Cu") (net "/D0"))
 (segment (start 53.81 75.4) (end 51.27 77.94) (width 0.25) (layer "B.Cu") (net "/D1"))
 (segment (start 51.27 77.94) (end 50 77.94) (width 0.25) (layer "B.Cu") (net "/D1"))
 (segment (start 53.81 77.94) (end 51.27 80.48) (width 0.25) (layer "B.Cu") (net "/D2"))
 (segment (start 51.27 80.48) (end 50 80.48) (width 0.25) (layer "B.Cu") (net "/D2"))
 (segment (start 66.51 83.02) (end 65.24 83.02) (width 0.25) (layer "B.Cu") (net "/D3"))
 (segment (start 69.05 80.48) (end 66.51 83.02) (width 0.25) (layer "B.Cu") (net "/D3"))
 (segment (start 66.51 80.48) (end 65.24 80.48) (width 0.25) (layer "B.Cu") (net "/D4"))
 (segment (start 69.05 77.94) (end 66.51 80.48) (width 0.25) (layer "B.Cu") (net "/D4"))
 (segment (start 67.78 75.4) (end 65.24 77.94) (width 0.25) (layer "B.Cu") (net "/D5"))
 (segment (start 69.05 75.4) (end 67.78 75.4) (width 0.25) (layer "B.Cu") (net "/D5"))
 (segment (start 66.51 75.4) (end 65.24 75.4) (width 0.25) (layer "B.Cu") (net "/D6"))
 (segment (start 69.05 72.86) (end 66.51 75.4) (width 0.25) (layer "B.Cu") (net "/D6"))
 (segment (start 69.05 70.32) (end 66.51 72.86) (width 0.25) (layer "B.Cu") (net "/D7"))
 (segment (start 66.51 72.86) (end 65.24 72.86) (width 0.25) (layer "B.Cu") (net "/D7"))
 (segment (start 71.7752 52.1473) (end 71.7752 51.4248) (width 0.25) (layer "F.Cu") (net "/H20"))
 (segment (start 70.2852 53.6373) (end 71.7752 52.1473) (width 0.25) (layer "F.Cu") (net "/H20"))
 (segment (start 70.2852 54.5683) (end 70.2852 53.6373) (width 0.25) (layer "F.Cu") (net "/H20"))
 (segment (start 68.5325 56.35) (end 69.5769 56.35) (width 0.25) (layer "F.Cu") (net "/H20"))
 (segment (start 71.7752 51.4248) (end 73.2 50) (width 0.25) (layer "F.Cu") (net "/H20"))
 (segment (start 69.5769 56.35) (end 70.8219 55.105) (width 0.25) (layer "F.Cu") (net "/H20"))
 (segment (start 70.8219 55.105) (end 70.2852 54.5683) (width 0.25) (layer "F.Cu") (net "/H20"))
 (segment (start 69.05 62.7) (end 67.7982 61.4482) (width 0.25) (layer "F.Cu") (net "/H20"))
 (segment (start 67.7982 57.0843) (end 68.5325 56.35) (width 0.25) (layer "F.Cu") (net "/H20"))
 (segment (start 67.7982 61.4482) (end 67.7982 57.0843) (width 0.25) (layer "F.Cu") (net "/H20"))
 (segment (start 65.242 65.24) (end 67.782 62.7) (width 0.25) (layer "B.Cu") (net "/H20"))
 (segment (start 65.24 65.24) (end 65.242 65.24) (width 0.25) (layer "B.Cu") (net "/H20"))
 (segment (start 67.782 62.7) (end 69.05 62.7) (width 0.25) (layer "B.Cu") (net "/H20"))
 (segment (start 74.4375 82.35) (end 74.84 81.9475) (width 0.25) (layer "F.Cu") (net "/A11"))
 (segment (start 74.84 81.9475) (end 74.84 79.45) (width 0.25) (layer "F.Cu") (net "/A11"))
 (segment (start 71.1717 78.3148) (end 71.0876 78.2307) (width 0.25) (layer "B.Cu") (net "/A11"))
 (segment (start 68.538 76.7048) (end 67.0228 78.22) (width 0.25) (layer "B.Cu") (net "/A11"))
 (segment (start 63.3735 77.8579) (end 64.7256 79.21) (width 0.25) (layer "B.Cu") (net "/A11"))
 (segment (start 74.7851 79.45) (end 73.6183 80.6168) (width 0.25) (layer "B.Cu") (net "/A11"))
 (segment (start 71.0876 76.7048) (end 68.538 76.7048) (width 0.25) (layer "B.Cu") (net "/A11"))
 (segment (start 74.84 79.45) (end 74.7851 79.45) (width 0.25) (layer "B.Cu") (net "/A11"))
 (segment (start 65.24 62.7) (end 65.0414 62.7) (width 0.25) (layer "B.Cu") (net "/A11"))
 (segment (start 70.8785 80.6168) (end 70.4013 80.1396) (width 0.25) (layer "B.Cu") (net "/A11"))
 (segment (start 70.4013 80.1396) (end 70.4013 79.0852) (width 0.25) (layer "B.Cu") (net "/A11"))
 (segment (start 64.7256 79.21) (end 66.0328 79.21) (width 0.25) (layer "B.Cu") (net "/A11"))
 (segment (start 73.6183 80.6168) (end 70.8785 80.6168) (width 0.25) (layer "B.Cu") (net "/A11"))
 (segment (start 65.0414 62.7) (end 63.3735 64.3679) (width 0.25) (layer "B.Cu") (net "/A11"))
 (segment (start 66.0328 79.21) (end 67.0228 78.22) (width 0.25) (layer "B.Cu") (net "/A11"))
 (segment (start 70.4013 79.0852) (end 71.1717 78.3148) (width 0.25) (layer "B.Cu") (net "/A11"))
 (segment (start 71.0876 78.2307) (end 71.0876 76.7048) (width 0.25) (layer "B.Cu") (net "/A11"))
 (segment (start 63.3735 64.3679) (end 63.3735 77.8579) (width 0.25) (layer "B.Cu") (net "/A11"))
 (segment (start 66.51 60.16) (end 65.24 60.16) (width 0.25) (layer "B.Cu") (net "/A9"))
 (segment (start 69.05 57.62) (end 66.51 60.16) (width 0.25) (layer "B.Cu") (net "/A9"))
 (segment (start 66.51 57.62) (end 65.24 57.62) (width 0.25) (layer "B.Cu") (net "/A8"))
 (segment (start 69.05 55.08) (end 66.51 57.62) (width 0.25) (layer "B.Cu") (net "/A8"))
 (segment (start 73.2057 72.7443) (end 72.3 73.65) (width 0.25) (layer "F.Cu") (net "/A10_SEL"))
 (segment (start 73.8468 72.7443) (end 73.2057 72.7443) (width 0.25) (layer "F.Cu") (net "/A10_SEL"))
 (segment (start 75.4987 70.4026) (end 75.4987 71.0924) (width 0.25) (layer "F.Cu") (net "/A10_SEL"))
 (segment (start 75.4987 62.9387) (end 75.4987 70.4026) (width 0.25) (layer "F.Cu") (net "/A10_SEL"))
 (segment (start 75.4987 71.0924) (end 73.8468 72.7443) (width 0.25) (layer "F.Cu") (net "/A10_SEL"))
 (segment (start 73.2 60.64) (end 75.4987 62.9387) (width 0.25) (layer "F.Cu") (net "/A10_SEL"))
 (segment (start 73.6783 64.6346) (end 74.4936 63.8193) (width 0.25) (layer "B.Cu") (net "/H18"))
 (segment (start 69.05 67.78) (end 71.9152 64.9148) (width 0.25) (layer "B.Cu") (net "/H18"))
 (segment (start 74.4936 63.8193) (end 74.4936 56.3736) (width 0.25) (layer "B.Cu") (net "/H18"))
 (segment (start 72.2575 64.9148) (end 72.3736 64.7987) (width 0.25) (layer "B.Cu") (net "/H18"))
 (segment (start 73.3989 64.7987) (end 73.563 64.6346) (width 0.25) (layer "B.Cu") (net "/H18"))
 (segment (start 74.4936 56.3736) (end 73.2 55.08) (width 0.25) (layer "B.Cu") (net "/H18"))
 (segment (start 72.3736 64.7987) (end 73.0026 64.7987) (width 0.25) (layer "B.Cu") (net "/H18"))
 (segment (start 73.563 64.6346) (end 73.6783 64.6346) (width 0.25) (layer "B.Cu") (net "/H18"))
 (segment (start 73.0026 64.7987) (end 73.3989 64.7987) (width 0.25) (layer "B.Cu") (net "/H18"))
 (segment (start 72.0934 64.9148) (end 72.2575 64.9148) (width 0.25) (layer "B.Cu") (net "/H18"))
 (segment (start 71.9152 64.9148) (end 72.0934 64.9148) (width 0.25) (layer "B.Cu") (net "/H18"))
 (segment (start 69.05 65.24) (end 69.052 65.24) (width 0.25) (layer "B.Cu") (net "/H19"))
 (segment (start 71.112 63.18) (end 73.2 63.18) (width 0.25) (layer "B.Cu") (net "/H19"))
 (segment (start 69.052 65.24) (end 71.112 63.18) (width 0.25) (layer "B.Cu") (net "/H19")))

